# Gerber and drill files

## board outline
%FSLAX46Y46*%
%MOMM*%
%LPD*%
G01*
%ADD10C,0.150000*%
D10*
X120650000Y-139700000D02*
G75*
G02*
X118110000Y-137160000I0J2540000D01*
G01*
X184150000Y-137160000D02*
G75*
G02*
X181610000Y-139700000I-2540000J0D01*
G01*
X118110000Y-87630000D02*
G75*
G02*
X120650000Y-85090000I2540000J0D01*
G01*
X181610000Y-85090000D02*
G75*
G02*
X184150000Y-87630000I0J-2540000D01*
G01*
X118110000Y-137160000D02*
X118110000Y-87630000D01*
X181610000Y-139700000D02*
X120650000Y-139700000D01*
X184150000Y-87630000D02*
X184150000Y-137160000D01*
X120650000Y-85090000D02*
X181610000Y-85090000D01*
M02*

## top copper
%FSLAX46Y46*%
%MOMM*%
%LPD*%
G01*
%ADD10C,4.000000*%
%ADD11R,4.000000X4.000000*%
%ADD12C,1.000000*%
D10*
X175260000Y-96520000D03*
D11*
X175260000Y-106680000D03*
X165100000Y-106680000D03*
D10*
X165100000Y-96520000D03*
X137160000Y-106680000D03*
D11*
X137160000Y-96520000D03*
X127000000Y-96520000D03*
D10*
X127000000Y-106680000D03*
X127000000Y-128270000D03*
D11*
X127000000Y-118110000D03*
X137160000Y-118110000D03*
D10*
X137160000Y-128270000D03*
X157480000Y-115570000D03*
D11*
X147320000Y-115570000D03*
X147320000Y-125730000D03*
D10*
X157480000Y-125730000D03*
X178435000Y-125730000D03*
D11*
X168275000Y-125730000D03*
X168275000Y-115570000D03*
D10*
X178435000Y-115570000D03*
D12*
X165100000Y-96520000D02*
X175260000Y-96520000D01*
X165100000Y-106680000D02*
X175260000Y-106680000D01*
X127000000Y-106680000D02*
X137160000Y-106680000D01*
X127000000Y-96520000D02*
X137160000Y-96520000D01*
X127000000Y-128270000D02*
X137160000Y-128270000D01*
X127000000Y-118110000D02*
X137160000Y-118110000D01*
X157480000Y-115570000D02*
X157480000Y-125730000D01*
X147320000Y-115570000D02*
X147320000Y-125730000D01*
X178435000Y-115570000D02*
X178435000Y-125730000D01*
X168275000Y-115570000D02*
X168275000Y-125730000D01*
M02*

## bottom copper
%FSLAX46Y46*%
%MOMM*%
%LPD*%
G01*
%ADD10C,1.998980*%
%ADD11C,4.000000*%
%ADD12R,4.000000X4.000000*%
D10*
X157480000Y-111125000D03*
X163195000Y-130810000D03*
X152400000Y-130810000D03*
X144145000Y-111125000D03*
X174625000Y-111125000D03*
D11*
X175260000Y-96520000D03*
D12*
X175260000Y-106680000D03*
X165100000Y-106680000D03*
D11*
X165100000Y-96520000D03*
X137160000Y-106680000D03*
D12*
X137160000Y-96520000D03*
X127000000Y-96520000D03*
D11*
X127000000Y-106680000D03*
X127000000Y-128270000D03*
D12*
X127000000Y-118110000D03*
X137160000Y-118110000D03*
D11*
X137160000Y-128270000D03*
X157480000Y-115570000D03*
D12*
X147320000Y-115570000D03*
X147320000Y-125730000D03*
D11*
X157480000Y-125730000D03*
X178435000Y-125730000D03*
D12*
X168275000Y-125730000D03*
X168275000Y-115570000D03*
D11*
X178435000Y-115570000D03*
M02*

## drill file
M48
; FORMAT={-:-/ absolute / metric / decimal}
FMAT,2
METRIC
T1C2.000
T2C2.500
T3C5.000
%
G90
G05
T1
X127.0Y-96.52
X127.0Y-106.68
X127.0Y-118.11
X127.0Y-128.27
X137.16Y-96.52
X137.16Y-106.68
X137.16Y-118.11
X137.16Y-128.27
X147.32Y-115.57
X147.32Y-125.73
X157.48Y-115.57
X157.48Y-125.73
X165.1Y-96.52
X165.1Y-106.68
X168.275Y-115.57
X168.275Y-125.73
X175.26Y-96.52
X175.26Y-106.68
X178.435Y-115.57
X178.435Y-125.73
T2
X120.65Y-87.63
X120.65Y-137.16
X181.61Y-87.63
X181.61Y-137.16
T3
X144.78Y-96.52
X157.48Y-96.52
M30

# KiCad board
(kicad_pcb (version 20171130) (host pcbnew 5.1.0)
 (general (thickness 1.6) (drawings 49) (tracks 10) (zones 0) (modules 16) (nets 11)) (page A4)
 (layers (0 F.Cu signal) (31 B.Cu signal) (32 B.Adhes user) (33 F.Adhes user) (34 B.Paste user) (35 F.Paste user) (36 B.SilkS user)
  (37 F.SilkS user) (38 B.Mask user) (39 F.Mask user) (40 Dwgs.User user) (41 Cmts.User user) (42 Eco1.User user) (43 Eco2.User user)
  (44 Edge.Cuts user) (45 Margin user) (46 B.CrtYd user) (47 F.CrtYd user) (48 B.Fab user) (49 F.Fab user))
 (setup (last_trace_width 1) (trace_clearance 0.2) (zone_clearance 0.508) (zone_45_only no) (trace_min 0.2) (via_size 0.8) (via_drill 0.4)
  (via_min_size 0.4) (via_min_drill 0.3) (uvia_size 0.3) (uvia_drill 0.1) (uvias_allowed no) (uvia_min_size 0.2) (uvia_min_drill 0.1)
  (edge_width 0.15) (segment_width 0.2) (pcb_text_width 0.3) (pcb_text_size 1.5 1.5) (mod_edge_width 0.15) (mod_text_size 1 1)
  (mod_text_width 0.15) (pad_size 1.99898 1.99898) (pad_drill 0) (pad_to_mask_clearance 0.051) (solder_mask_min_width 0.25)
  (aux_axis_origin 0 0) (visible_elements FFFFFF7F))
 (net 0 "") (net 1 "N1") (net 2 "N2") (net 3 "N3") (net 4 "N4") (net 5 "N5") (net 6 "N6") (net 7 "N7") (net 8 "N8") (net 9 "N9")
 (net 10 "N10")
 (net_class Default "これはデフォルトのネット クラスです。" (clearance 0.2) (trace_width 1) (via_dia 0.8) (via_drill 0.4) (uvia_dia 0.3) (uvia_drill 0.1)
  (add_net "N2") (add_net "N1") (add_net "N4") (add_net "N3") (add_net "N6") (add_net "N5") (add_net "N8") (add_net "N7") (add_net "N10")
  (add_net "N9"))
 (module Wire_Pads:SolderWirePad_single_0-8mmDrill (layer B.Cu) (at 157.48 111.125)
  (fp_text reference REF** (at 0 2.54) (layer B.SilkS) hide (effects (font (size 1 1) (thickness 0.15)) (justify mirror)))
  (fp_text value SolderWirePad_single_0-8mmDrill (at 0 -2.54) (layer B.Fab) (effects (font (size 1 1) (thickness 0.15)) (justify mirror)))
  (pad 1 smd circle (at 0 0) (size 1.99898 1.99898) (layers B.Cu B.Paste B.Mask)))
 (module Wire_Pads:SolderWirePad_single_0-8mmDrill (layer B.Cu) (at 163.195 130.81)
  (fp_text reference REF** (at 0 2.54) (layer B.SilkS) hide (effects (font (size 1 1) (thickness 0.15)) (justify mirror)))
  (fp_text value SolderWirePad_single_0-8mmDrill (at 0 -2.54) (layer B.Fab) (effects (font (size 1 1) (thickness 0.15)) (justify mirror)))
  (pad 1 smd circle (at 0 0) (size 1.99898 1.99898) (layers B.Cu B.Paste B.Mask)))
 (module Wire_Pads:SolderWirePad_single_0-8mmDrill (layer B.Cu) (at 152.4 130.81)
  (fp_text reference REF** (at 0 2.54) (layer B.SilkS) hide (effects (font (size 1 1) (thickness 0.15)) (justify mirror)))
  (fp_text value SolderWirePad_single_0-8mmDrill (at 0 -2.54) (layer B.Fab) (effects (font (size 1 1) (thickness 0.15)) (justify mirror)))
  (pad 1 smd circle (at 0 0) (size 1.99898 1.99898) (layers B.Cu B.Paste B.Mask)))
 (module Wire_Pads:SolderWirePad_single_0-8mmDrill (layer B.Cu) (at 144.145 111.125)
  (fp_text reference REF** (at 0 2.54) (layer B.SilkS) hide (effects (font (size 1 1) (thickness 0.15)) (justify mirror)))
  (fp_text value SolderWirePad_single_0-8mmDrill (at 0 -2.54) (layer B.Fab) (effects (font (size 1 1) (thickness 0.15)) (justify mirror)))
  (pad 1 smd circle (at 0 0) (size 1.99898 1.99898) (layers B.Cu B.Paste B.Mask)))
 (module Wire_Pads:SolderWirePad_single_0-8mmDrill (layer B.Cu) (at 174.625 111.125)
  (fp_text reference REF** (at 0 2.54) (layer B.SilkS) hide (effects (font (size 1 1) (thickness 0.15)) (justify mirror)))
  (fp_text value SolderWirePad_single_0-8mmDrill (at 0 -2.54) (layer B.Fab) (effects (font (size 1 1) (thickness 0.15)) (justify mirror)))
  (pad 1 smd circle (at 0 0) (size 1.99898 1.99898) (layers B.Cu B.Paste B.Mask)))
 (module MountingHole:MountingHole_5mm (layer F.Cu) (at 144.78 96.52)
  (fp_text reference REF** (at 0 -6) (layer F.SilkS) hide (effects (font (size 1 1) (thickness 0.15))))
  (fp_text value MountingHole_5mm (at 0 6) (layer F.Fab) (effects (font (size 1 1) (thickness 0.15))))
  (pad 1 np_thru_hole circle (at 0 0) (size 5 5) (drill 5) (layers *.Cu *.Mask)))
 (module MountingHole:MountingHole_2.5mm (layer F.Cu) (at 120.65 87.63)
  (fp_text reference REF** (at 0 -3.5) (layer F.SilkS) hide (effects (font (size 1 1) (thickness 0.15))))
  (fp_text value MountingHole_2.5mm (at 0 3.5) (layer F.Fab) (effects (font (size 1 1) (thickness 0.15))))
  (pad 1 np_thru_hole circle (at 0 0) (size 2.5 2.5) (drill 2.5) (layers *.Cu *.Mask)))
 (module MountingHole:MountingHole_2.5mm (layer F.Cu) (at 181.61 87.63)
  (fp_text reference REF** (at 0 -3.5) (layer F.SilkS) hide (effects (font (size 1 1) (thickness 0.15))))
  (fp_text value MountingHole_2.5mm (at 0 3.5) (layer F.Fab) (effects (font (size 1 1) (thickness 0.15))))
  (pad 1 np_thru_hole circle (at 0 0) (size 2.5 2.5) (drill 2.5) (layers *.Cu *.Mask)))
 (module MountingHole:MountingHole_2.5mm (layer F.Cu) (at 120.65 137.16)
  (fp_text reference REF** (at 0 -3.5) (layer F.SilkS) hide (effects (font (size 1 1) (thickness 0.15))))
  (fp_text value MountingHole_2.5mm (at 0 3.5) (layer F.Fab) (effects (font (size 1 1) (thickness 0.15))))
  (pad 1 np_thru_hole circle (at 0 0) (size 2.5 2.5) (drill 2.5) (layers *.Cu *.Mask)))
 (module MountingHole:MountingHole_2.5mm (layer F.Cu) (at 181.61 137.16)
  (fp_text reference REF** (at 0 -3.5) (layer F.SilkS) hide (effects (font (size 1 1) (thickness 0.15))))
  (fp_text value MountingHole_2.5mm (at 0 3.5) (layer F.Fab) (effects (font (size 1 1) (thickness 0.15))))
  (pad 1 np_thru_hole circle (at 0 0) (size 2.5 2.5) (drill 2.5) (layers *.Cu *.Mask)))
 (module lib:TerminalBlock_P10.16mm (layer F.Cu) (at 175.26 106.68 90)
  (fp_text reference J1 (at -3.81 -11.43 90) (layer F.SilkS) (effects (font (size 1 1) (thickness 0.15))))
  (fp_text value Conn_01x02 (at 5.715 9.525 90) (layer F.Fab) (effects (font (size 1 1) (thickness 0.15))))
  (pad 2 thru_hole circle (at 10.16 0 90) (size 4 4) (drill 2) (layers *.Cu *.Mask) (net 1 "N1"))
  (pad 1 thru_hole rect (at 0 0 90) (size 4 4) (drill 2) (layers *.Cu *.Mask) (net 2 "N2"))
  (pad 1 thru_hole rect (at 0 -10.16 90) (size 4 4) (drill 2) (layers *.Cu *.Mask) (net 2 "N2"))
  (pad 2 thru_hole circle (at 10.16 -10.16 90) (size 4 4) (drill 2) (layers *.Cu *.Mask) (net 1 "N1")))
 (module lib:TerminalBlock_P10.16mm (layer F.Cu) (at 127 96.52 270)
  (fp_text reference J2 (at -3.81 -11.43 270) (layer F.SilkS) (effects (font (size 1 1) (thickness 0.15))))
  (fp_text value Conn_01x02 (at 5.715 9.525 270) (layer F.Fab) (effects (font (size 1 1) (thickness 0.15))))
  (pad 2 thru_hole circle (at 10.16 -10.16 270) (size 4 4) (drill 2) (layers *.Cu *.Mask) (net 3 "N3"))
  (pad 1 thru_hole rect (at 0 -10.16 270) (size 4 4) (drill 2) (layers *.Cu *.Mask) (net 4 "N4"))
  (pad 1 thru_hole rect (at 0 0 270) (size 4 4) (drill 2) (layers *.Cu *.Mask) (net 4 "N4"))
  (pad 2 thru_hole circle (at 10.16 0 270) (size 4 4) (drill 2) (layers *.Cu *.Mask) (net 3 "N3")))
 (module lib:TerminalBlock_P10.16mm (layer F.Cu) (at 127 118.11 270)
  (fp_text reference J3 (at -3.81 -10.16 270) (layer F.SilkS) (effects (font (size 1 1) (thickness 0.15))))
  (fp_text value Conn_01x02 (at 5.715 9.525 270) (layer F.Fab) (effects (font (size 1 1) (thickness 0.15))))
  (pad 2 thru_hole circle (at 10.16 0 270) (size 4 4) (drill 2) (layers *.Cu *.Mask) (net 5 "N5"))
  (pad 1 thru_hole rect (at 0 0 270) (size 4 4) (drill 2) (layers *.Cu *.Mask) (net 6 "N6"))
  (pad 1 thru_hole rect (at 0 -10.16 270) (size 4 4) (drill 2) (layers *.Cu *.Mask) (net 6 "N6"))
  (pad 2 thru_hole circle (at 10.16 -10.16 270) (size 4 4) (drill 2) (layers *.Cu *.Mask) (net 5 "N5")))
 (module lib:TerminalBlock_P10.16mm (layer F.Cu) (at 147.32 125.73)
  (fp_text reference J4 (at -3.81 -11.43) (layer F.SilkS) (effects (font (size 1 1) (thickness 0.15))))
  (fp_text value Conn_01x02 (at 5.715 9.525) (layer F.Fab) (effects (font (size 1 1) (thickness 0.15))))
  (pad 2 thru_hole circle (at 10.16 -10.16) (size 4 4) (drill 2) (layers *.Cu *.Mask) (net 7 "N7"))
  (pad 1 thru_hole rect (at 0 -10.16) (size 4 4) (drill 2) (layers *.Cu *.Mask) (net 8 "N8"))
  (pad 1 thru_hole rect (at 0 0) (size 4 4) (drill 2) (layers *.Cu *.Mask) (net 8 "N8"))
  (pad 2 thru_hole circle (at 10.16 0) (size 4 4) (drill 2) (layers *.Cu *.Mask) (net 7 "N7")))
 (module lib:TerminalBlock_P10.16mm (layer F.Cu) (at 168.275 125.73)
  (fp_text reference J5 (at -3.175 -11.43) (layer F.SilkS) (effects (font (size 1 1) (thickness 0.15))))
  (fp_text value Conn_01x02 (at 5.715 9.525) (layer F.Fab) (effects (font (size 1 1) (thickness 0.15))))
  (pad 2 thru_hole circle (at 10.16 0) (size 4 4) (drill 2) (layers *.Cu *.Mask) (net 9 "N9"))
  (pad 1 thru_hole rect (at 0 0) (size 4 4) (drill 2) (layers *.Cu *.Mask) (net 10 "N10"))
  (pad 1 thru_hole rect (at 0 -10.16) (size 4 4) (drill 2) (layers *.Cu *.Mask) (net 10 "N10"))
  (pad 2 thru_hole circle (at 10.16 -10.16) (size 4 4) (drill 2) (layers *.Cu *.Mask) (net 9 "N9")))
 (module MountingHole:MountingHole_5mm (layer F.Cu) (at 157.48 96.52)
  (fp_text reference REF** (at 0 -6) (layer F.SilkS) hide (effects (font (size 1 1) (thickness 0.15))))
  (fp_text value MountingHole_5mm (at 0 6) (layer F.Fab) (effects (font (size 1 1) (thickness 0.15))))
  (pad 1 np_thru_hole circle (at 0 0) (size 5 5) (drill 5) (layers *.Cu *.Mask)))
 (gr_arc (start 120.65 137.16) (end 118.11 137.16) (angle -90) (layer Edge.Cuts) (width 0.15))
 (gr_arc (start 181.61 137.16) (end 181.61 139.7) (angle -90) (layer Edge.Cuts) (width 0.15))
 (gr_arc (start 120.65 87.63) (end 120.65 85.09) (angle -90) (layer Edge.Cuts) (width 0.15))
 (gr_arc (start 181.61 87.63) (end 184.15 87.63) (angle -90) (layer Edge.Cuts) (width 0.15))
 (gr_line (start 118.11 137.16) (end 118.11 87.63) (layer Edge.Cuts) (width 0.15))
 (gr_line (start 181.61 139.7) (end 120.65 139.7) (layer Edge.Cuts) (width 0.15))
 (gr_line (start 184.15 87.63) (end 184.15 137.16) (layer Edge.Cuts) (width 0.15))
 (gr_line (start 120.65 85.09) (end 181.61 85.09) (layer Edge.Cuts) (width 0.15))
 (segment (start 165.1 96.52) (end 175.26 96.52) (width 1) (layer F.Cu) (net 1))
 (segment (start 165.1 106.68) (end 175.26 106.68) (width 1) (layer F.Cu) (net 2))
 (segment (start 127 106.68) (end 137.16 106.68) (width 1) (layer F.Cu) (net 3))
 (segment (start 127 96.52) (end 137.16 96.52) (width 1) (layer F.Cu) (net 4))
 (segment (start 127 128.27) (end 137.16 128.27) (width 1) (layer F.Cu) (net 5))
 (segment (start 127 118.11) (end 137.16 118.11) (width 1) (layer F.Cu) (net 6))
 (segment (start 157.48 115.57) (end 157.48 125.73) (width 1) (layer F.Cu) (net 7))
 (segment (start 147.32 115.57) (end 147.32 125.73) (width 1) (layer F.Cu) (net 8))
 (segment (start 178.435 115.57) (end 178.435 125.73) (width 1) (layer F.Cu) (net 9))
 (segment (start 168.275 115.57) (end 168.275 125.73) (width 1) (layer F.Cu) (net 10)))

